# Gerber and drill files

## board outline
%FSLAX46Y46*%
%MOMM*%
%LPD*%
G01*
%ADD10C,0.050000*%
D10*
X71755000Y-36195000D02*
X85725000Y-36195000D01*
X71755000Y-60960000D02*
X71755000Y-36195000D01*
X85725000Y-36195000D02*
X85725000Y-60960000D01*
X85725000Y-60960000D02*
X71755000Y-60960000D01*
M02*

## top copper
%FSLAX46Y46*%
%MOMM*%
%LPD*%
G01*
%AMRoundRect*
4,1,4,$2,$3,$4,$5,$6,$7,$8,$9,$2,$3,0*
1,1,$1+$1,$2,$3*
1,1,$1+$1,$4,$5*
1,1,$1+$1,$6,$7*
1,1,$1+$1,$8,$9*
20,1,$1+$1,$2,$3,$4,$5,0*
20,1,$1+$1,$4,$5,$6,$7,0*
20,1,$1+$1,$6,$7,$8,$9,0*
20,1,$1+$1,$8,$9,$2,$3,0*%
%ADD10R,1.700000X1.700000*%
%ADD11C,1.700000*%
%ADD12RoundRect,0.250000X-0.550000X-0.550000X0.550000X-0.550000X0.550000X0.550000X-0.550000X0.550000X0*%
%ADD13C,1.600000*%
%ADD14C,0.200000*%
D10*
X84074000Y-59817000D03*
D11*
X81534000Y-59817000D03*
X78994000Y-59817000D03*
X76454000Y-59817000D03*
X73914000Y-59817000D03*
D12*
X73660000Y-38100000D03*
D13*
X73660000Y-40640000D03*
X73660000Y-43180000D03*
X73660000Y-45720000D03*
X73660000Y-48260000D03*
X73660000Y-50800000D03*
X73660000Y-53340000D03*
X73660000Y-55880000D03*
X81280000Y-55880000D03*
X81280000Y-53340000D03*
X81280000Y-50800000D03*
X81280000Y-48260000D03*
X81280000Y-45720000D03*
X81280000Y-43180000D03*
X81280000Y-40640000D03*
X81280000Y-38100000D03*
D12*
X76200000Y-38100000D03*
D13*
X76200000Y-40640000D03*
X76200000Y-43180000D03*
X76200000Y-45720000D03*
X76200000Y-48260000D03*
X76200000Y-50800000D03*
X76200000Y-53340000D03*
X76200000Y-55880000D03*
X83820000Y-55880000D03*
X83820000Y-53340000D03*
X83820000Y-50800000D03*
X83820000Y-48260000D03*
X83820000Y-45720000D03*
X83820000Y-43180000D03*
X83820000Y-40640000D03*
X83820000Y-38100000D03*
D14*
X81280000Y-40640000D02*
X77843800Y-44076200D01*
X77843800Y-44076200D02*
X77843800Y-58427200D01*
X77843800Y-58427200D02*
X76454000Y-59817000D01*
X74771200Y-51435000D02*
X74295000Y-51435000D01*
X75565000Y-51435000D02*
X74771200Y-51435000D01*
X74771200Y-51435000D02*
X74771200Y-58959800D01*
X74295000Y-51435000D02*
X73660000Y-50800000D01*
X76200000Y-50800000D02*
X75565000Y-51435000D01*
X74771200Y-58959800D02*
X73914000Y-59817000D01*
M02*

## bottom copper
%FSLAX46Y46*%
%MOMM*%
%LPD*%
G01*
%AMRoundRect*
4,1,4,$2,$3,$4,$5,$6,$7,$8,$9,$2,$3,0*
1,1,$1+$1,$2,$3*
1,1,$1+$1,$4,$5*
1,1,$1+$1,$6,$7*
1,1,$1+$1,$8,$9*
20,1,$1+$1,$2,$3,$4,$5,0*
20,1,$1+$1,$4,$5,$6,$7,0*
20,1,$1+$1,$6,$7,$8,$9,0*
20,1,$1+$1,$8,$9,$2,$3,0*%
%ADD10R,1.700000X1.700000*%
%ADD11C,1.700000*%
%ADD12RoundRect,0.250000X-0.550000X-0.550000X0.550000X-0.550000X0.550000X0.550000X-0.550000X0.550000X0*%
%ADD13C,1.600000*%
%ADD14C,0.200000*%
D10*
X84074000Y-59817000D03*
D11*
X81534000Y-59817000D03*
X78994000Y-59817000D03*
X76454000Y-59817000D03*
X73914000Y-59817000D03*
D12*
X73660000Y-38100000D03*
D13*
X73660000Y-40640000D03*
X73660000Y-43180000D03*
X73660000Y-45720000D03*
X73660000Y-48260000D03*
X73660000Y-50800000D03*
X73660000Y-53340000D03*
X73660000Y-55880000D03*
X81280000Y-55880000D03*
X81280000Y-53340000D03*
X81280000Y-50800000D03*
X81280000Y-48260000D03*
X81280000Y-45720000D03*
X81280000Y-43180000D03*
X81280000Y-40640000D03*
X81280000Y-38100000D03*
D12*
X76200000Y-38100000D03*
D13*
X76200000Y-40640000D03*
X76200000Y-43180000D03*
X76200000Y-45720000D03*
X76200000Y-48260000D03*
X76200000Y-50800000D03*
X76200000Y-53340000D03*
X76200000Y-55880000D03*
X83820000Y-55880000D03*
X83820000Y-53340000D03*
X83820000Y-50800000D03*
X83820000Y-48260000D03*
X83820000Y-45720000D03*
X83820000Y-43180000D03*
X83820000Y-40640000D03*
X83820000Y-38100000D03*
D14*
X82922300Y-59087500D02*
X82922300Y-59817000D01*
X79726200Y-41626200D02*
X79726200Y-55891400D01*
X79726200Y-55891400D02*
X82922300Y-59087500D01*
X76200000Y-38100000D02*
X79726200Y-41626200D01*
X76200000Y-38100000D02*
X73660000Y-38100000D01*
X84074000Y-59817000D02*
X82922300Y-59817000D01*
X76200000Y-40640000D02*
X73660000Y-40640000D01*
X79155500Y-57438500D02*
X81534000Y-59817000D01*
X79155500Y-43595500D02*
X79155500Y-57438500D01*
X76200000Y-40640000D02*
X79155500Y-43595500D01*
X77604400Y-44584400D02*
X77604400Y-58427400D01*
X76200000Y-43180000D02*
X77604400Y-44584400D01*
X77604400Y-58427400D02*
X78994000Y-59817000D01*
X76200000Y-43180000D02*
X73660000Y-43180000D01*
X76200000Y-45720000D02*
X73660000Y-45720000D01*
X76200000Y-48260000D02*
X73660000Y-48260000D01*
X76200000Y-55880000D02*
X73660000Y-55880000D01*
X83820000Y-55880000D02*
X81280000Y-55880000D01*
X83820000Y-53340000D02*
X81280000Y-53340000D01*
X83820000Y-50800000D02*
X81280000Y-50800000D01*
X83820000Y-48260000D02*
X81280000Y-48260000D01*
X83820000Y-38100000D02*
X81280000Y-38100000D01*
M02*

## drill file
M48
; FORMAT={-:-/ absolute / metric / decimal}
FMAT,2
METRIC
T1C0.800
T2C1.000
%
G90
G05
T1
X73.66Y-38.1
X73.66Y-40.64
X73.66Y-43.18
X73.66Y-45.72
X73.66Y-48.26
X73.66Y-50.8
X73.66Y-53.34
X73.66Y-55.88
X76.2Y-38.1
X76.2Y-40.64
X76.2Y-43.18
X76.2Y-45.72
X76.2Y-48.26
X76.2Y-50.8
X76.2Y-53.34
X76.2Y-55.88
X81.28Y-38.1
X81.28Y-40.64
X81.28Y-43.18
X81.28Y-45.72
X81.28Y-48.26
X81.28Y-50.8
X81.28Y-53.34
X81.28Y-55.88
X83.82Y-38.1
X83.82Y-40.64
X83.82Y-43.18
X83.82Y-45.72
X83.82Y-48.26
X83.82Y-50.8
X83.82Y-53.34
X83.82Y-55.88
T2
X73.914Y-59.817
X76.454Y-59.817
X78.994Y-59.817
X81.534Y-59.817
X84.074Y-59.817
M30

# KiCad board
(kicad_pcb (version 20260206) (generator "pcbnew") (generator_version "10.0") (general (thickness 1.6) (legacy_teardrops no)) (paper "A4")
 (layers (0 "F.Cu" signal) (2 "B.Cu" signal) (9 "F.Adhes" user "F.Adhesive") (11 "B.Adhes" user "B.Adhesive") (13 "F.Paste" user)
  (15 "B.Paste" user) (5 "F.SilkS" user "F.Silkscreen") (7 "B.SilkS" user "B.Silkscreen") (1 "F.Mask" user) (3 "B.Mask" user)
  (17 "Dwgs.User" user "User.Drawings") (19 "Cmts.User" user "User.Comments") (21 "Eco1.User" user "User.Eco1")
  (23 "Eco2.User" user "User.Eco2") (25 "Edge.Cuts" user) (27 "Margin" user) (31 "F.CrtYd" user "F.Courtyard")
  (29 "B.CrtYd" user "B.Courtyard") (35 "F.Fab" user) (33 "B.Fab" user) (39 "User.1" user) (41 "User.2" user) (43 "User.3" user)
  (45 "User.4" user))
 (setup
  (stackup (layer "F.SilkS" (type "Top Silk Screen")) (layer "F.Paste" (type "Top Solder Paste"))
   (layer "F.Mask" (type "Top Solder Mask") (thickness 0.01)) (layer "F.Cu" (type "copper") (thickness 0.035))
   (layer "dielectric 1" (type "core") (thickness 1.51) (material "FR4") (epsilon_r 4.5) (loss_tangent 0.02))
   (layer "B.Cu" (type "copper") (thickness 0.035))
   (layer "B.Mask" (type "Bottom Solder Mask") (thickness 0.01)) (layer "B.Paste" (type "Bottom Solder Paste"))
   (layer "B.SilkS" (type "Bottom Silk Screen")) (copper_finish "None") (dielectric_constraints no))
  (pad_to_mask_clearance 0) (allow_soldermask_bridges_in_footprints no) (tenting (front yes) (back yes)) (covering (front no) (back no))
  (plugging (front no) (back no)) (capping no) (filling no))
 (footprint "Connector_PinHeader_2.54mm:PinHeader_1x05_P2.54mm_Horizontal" (layer "F.Cu") (at 84.074 59.817 -90)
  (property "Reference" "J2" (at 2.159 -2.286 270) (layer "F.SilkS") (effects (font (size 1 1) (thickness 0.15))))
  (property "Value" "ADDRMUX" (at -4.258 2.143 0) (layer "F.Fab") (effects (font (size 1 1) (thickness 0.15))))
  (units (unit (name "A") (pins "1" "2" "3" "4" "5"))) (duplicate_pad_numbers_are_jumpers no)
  (pad "1" thru_hole rect (at 0 0 270) (size 1.7 1.7) (drill 1) (layers "*.Cu" "*.Mask") (remove_unused_layers no) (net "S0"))
  (pad "2" thru_hole circle (at 0 2.54 270) (size 1.7 1.7) (drill 1) (layers "*.Cu" "*.Mask") (remove_unused_layers no) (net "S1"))
  (pad "3" thru_hole circle (at 0 5.08 270) (size 1.7 1.7) (drill 1) (layers "*.Cu" "*.Mask") (remove_unused_layers no) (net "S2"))
  (pad "4" thru_hole circle (at 0 7.62 270) (size 1.7 1.7) (drill 1) (layers "*.Cu" "*.Mask") (remove_unused_layers no) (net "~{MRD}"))
  (pad "5" thru_hole circle (at 0 10.16 270) (size 1.7 1.7) (drill 1) (layers "*.Cu" "*.Mask") (remove_unused_layers no) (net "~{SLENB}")))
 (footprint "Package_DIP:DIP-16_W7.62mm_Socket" (layer "F.Cu") (at 73.66 38.1)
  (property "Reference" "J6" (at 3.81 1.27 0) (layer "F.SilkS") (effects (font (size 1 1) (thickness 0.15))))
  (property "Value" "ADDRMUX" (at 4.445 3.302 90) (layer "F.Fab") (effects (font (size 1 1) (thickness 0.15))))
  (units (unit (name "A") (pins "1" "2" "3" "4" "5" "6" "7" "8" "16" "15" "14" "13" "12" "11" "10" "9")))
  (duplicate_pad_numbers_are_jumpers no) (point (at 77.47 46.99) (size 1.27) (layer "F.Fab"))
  (pad "1" thru_hole roundrect (at 0 0) (size 1.6 1.6) (drill 0.8) (layers "*.Cu" "*.Mask") (remove_unused_layers no)
   (roundrect_rratio 0.15625) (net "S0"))
  (pad "2" thru_hole circle (at 0 2.54) (size 1.6 1.6) (drill 0.8) (layers "*.Cu" "*.Mask") (remove_unused_layers no) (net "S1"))
  (pad "3" thru_hole circle (at 0 5.08) (size 1.6 1.6) (drill 0.8) (layers "*.Cu" "*.Mask") (remove_unused_layers no) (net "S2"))
  (pad "4" thru_hole circle (at 0 7.62) (size 1.6 1.6) (drill 0.8) (layers "*.Cu" "*.Mask") (remove_unused_layers no) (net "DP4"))
  (pad "5" thru_hole circle (at 0 10.16) (size 1.6 1.6) (drill 0.8) (layers "*.Cu" "*.Mask") (remove_unused_layers no) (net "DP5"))
  (pad "6" thru_hole circle (at 0 12.7) (size 1.6 1.6) (drill 0.8) (layers "*.Cu" "*.Mask") (remove_unused_layers no) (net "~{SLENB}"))
  (pad "7" thru_hole circle (at 0 15.24) (size 1.6 1.6) (drill 0.8) (layers "*.Cu" "*.Mask") (remove_unused_layers no)
   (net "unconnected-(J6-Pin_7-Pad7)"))
  (pad "8" thru_hole circle (at 0 17.78) (size 1.6 1.6) (drill 0.8) (layers "*.Cu" "*.Mask") (remove_unused_layers no) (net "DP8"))
  (pad "9" thru_hole circle (at 7.62 17.78) (size 1.6 1.6) (drill 0.8) (layers "*.Cu" "*.Mask") (remove_unused_layers no) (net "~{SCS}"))
  (pad "10" thru_hole circle (at 7.62 15.24) (size 1.6 1.6) (drill 0.8) (layers "*.Cu" "*.Mask") (remove_unused_layers no) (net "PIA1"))
  (pad "11" thru_hole circle (at 7.62 12.7) (size 1.6 1.6) (drill 0.8) (layers "*.Cu" "*.Mask") (remove_unused_layers no) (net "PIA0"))
  (pad "12" thru_hole circle (at 7.62 10.16) (size 1.6 1.6) (drill 0.8) (layers "*.Cu" "*.Mask") (remove_unused_layers no) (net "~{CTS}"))
  (pad "13" thru_hole circle (at 7.62 7.62) (size 1.6 1.6) (drill 0.8) (layers "*.Cu" "*.Mask") (remove_unused_layers no) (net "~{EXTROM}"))
  (pad "14" thru_hole circle (at 7.62 5.08) (size 1.6 1.6) (drill 0.8) (layers "*.Cu" "*.Mask") (remove_unused_layers no) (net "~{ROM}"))
  (pad "15" thru_hole circle (at 7.62 2.54) (size 1.6 1.6) (drill 0.8) (layers "*.Cu" "*.Mask") (remove_unused_layers no) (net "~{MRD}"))
  (pad "16" thru_hole circle (at 7.62 0) (size 1.6 1.6) (drill 0.8) (layers "*.Cu" "*.Mask") (remove_unused_layers no) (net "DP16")))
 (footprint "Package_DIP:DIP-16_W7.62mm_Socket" (layer "F.Cu") (at 76.2 38.1)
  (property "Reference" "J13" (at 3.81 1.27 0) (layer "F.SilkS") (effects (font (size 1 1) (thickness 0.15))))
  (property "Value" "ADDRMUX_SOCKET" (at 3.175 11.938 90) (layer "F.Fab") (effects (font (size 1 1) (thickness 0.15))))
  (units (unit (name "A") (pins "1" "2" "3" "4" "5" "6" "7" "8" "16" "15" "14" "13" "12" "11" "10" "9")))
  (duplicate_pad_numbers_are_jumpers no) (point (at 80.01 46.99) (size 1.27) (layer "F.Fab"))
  (pad "1" thru_hole roundrect (at 0 0) (size 1.6 1.6) (drill 0.8) (layers "*.Cu" "*.Mask") (remove_unused_layers no)
   (roundrect_rratio 0.15625) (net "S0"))
  (pad "2" thru_hole circle (at 0 2.54) (size 1.6 1.6) (drill 0.8) (layers "*.Cu" "*.Mask") (remove_unused_layers no) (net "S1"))
  (pad "3" thru_hole circle (at 0 5.08) (size 1.6 1.6) (drill 0.8) (layers "*.Cu" "*.Mask") (remove_unused_layers no) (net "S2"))
  (pad "4" thru_hole circle (at 0 7.62) (size 1.6 1.6) (drill 0.8) (layers "*.Cu" "*.Mask") (remove_unused_layers no) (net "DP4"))
  (pad "5" thru_hole circle (at 0 10.16) (size 1.6 1.6) (drill 0.8) (layers "*.Cu" "*.Mask") (remove_unused_layers no) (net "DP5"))
  (pad "6" thru_hole circle (at 0 12.7) (size 1.6 1.6) (drill 0.8) (layers "*.Cu" "*.Mask") (remove_unused_layers no) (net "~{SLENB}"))
  (pad "7" thru_hole circle (at 0 15.24) (size 1.6 1.6) (drill 0.8) (layers "*.Cu" "*.Mask") (remove_unused_layers no)
   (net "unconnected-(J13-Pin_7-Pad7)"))
  (pad "8" thru_hole circle (at 0 17.78) (size 1.6 1.6) (drill 0.8) (layers "*.Cu" "*.Mask") (remove_unused_layers no) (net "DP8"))
  (pad "9" thru_hole circle (at 7.62 17.78) (size 1.6 1.6) (drill 0.8) (layers "*.Cu" "*.Mask") (remove_unused_layers no) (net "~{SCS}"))
  (pad "10" thru_hole circle (at 7.62 15.24) (size 1.6 1.6) (drill 0.8) (layers "*.Cu" "*.Mask") (remove_unused_layers no) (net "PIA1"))
  (pad "11" thru_hole circle (at 7.62 12.7) (size 1.6 1.6) (drill 0.8) (layers "*.Cu" "*.Mask") (remove_unused_layers no) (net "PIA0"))
  (pad "12" thru_hole circle (at 7.62 10.16) (size 1.6 1.6) (drill 0.8) (layers "*.Cu" "*.Mask") (remove_unused_layers no) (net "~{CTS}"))
  (pad "13" thru_hole circle (at 7.62 7.62) (size 1.6 1.6) (drill 0.8) (layers "*.Cu" "*.Mask") (remove_unused_layers no)
   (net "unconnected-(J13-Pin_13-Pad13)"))
  (pad "14" thru_hole circle (at 7.62 5.08) (size 1.6 1.6) (drill 0.8) (layers "*.Cu" "*.Mask") (remove_unused_layers no)
   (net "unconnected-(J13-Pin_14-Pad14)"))
  (pad "15" thru_hole circle (at 7.62 2.54) (size 1.6 1.6) (drill 0.8) (layers "*.Cu" "*.Mask") (remove_unused_layers no)
   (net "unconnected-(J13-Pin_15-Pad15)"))
  (pad "16" thru_hole circle (at 7.62 0) (size 1.6 1.6) (drill 0.8) (layers "*.Cu" "*.Mask") (remove_unused_layers no) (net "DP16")))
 (gr_line (start 71.755 36.195) (end 85.725 36.195) (stroke (width 0.05) (type default)) (layer "Edge.Cuts"))
 (gr_line (start 71.755 60.96) (end 71.755 36.195) (stroke (width 0.05) (type default)) (layer "Edge.Cuts"))
 (gr_line (start 85.725 36.195) (end 85.725 60.96) (stroke (width 0.05) (type default)) (layer "Edge.Cuts"))
 (gr_line (start 85.725 60.96) (end 71.755 60.96) (stroke (width 0.05) (type default)) (layer "Edge.Cuts"))
 (segment (start 82.9223 59.0875) (end 82.9223 59.817) (width 0.2) (layer "B.Cu") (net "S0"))
 (segment (start 79.7262 41.6262) (end 79.7262 55.8914) (width 0.2) (layer "B.Cu") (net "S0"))
 (segment (start 79.7262 55.8914) (end 82.9223 59.0875) (width 0.2) (layer "B.Cu") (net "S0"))
 (segment (start 76.2 38.1) (end 79.7262 41.6262) (width 0.2) (layer "B.Cu") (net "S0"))
 (segment (start 76.2 38.1) (end 73.66 38.1) (width 0.2) (layer "B.Cu") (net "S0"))
 (segment (start 84.074 59.817) (end 82.9223 59.817) (width 0.2) (layer "B.Cu") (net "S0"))
 (segment (start 76.2 40.64) (end 73.66 40.64) (width 0.2) (layer "B.Cu") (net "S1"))
 (segment (start 79.1555 57.4385) (end 81.534 59.817) (width 0.2) (layer "B.Cu") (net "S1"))
 (segment (start 79.1555 43.5955) (end 79.1555 57.4385) (width 0.2) (layer "B.Cu") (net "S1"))
 (segment (start 76.2 40.64) (end 79.1555 43.5955) (width 0.2) (layer "B.Cu") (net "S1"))
 (segment (start 77.6044 44.5844) (end 77.6044 58.4274) (width 0.2) (layer "B.Cu") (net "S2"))
 (segment (start 76.2 43.18) (end 77.6044 44.5844) (width 0.2) (layer "B.Cu") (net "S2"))
 (segment (start 77.6044 58.4274) (end 78.994 59.817) (width 0.2) (layer "B.Cu") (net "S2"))
 (segment (start 76.2 43.18) (end 73.66 43.18) (width 0.2) (layer "B.Cu") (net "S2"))
 (segment (start 81.28 40.64) (end 77.8438 44.0762) (width 0.2) (layer "F.Cu") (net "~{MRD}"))
 (segment (start 77.8438 44.0762) (end 77.8438 58.4272) (width 0.2) (layer "F.Cu") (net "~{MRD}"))
 (segment (start 77.8438 58.4272) (end 76.454 59.817) (width 0.2) (layer "F.Cu") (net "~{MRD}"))
 (segment (start 74.7712 51.435) (end 74.295 51.435) (width 0.2) (layer "F.Cu") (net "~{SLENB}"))
 (segment (start 75.565 51.435) (end 74.7712 51.435) (width 0.2) (layer "F.Cu") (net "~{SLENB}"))
 (segment (start 74.7712 51.435) (end 74.7712 58.9598) (width 0.2) (layer "F.Cu") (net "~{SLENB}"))
 (segment (start 74.295 51.435) (end 73.66 50.8) (width 0.2) (layer "F.Cu") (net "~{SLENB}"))
 (segment (start 76.2 50.8) (end 75.565 51.435) (width 0.2) (layer "F.Cu") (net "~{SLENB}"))
 (segment (start 74.7712 58.9598) (end 73.914 59.817) (width 0.2) (layer "F.Cu") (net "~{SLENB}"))
 (segment (start 76.2 45.72) (end 73.66 45.72) (width 0.2) (layer "B.Cu") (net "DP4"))
 (segment (start 76.2 48.26) (end 73.66 48.26) (width 0.2) (layer "B.Cu") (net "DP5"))
 (segment (start 76.2 55.88) (end 73.66 55.88) (width 0.2) (layer "B.Cu") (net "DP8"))
 (segment (start 83.82 55.88) (end 81.28 55.88) (width 0.2) (layer "B.Cu") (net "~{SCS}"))
 (segment (start 83.82 53.34) (end 81.28 53.34) (width 0.2) (layer "B.Cu") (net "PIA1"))
 (segment (start 83.82 50.8) (end 81.28 50.8) (width 0.2) (layer "B.Cu") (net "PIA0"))
 (segment (start 83.82 48.26) (end 81.28 48.26) (width 0.2) (layer "B.Cu") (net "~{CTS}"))
 (segment (start 83.82 38.1) (end 81.28 38.1) (width 0.2) (layer "B.Cu") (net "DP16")))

